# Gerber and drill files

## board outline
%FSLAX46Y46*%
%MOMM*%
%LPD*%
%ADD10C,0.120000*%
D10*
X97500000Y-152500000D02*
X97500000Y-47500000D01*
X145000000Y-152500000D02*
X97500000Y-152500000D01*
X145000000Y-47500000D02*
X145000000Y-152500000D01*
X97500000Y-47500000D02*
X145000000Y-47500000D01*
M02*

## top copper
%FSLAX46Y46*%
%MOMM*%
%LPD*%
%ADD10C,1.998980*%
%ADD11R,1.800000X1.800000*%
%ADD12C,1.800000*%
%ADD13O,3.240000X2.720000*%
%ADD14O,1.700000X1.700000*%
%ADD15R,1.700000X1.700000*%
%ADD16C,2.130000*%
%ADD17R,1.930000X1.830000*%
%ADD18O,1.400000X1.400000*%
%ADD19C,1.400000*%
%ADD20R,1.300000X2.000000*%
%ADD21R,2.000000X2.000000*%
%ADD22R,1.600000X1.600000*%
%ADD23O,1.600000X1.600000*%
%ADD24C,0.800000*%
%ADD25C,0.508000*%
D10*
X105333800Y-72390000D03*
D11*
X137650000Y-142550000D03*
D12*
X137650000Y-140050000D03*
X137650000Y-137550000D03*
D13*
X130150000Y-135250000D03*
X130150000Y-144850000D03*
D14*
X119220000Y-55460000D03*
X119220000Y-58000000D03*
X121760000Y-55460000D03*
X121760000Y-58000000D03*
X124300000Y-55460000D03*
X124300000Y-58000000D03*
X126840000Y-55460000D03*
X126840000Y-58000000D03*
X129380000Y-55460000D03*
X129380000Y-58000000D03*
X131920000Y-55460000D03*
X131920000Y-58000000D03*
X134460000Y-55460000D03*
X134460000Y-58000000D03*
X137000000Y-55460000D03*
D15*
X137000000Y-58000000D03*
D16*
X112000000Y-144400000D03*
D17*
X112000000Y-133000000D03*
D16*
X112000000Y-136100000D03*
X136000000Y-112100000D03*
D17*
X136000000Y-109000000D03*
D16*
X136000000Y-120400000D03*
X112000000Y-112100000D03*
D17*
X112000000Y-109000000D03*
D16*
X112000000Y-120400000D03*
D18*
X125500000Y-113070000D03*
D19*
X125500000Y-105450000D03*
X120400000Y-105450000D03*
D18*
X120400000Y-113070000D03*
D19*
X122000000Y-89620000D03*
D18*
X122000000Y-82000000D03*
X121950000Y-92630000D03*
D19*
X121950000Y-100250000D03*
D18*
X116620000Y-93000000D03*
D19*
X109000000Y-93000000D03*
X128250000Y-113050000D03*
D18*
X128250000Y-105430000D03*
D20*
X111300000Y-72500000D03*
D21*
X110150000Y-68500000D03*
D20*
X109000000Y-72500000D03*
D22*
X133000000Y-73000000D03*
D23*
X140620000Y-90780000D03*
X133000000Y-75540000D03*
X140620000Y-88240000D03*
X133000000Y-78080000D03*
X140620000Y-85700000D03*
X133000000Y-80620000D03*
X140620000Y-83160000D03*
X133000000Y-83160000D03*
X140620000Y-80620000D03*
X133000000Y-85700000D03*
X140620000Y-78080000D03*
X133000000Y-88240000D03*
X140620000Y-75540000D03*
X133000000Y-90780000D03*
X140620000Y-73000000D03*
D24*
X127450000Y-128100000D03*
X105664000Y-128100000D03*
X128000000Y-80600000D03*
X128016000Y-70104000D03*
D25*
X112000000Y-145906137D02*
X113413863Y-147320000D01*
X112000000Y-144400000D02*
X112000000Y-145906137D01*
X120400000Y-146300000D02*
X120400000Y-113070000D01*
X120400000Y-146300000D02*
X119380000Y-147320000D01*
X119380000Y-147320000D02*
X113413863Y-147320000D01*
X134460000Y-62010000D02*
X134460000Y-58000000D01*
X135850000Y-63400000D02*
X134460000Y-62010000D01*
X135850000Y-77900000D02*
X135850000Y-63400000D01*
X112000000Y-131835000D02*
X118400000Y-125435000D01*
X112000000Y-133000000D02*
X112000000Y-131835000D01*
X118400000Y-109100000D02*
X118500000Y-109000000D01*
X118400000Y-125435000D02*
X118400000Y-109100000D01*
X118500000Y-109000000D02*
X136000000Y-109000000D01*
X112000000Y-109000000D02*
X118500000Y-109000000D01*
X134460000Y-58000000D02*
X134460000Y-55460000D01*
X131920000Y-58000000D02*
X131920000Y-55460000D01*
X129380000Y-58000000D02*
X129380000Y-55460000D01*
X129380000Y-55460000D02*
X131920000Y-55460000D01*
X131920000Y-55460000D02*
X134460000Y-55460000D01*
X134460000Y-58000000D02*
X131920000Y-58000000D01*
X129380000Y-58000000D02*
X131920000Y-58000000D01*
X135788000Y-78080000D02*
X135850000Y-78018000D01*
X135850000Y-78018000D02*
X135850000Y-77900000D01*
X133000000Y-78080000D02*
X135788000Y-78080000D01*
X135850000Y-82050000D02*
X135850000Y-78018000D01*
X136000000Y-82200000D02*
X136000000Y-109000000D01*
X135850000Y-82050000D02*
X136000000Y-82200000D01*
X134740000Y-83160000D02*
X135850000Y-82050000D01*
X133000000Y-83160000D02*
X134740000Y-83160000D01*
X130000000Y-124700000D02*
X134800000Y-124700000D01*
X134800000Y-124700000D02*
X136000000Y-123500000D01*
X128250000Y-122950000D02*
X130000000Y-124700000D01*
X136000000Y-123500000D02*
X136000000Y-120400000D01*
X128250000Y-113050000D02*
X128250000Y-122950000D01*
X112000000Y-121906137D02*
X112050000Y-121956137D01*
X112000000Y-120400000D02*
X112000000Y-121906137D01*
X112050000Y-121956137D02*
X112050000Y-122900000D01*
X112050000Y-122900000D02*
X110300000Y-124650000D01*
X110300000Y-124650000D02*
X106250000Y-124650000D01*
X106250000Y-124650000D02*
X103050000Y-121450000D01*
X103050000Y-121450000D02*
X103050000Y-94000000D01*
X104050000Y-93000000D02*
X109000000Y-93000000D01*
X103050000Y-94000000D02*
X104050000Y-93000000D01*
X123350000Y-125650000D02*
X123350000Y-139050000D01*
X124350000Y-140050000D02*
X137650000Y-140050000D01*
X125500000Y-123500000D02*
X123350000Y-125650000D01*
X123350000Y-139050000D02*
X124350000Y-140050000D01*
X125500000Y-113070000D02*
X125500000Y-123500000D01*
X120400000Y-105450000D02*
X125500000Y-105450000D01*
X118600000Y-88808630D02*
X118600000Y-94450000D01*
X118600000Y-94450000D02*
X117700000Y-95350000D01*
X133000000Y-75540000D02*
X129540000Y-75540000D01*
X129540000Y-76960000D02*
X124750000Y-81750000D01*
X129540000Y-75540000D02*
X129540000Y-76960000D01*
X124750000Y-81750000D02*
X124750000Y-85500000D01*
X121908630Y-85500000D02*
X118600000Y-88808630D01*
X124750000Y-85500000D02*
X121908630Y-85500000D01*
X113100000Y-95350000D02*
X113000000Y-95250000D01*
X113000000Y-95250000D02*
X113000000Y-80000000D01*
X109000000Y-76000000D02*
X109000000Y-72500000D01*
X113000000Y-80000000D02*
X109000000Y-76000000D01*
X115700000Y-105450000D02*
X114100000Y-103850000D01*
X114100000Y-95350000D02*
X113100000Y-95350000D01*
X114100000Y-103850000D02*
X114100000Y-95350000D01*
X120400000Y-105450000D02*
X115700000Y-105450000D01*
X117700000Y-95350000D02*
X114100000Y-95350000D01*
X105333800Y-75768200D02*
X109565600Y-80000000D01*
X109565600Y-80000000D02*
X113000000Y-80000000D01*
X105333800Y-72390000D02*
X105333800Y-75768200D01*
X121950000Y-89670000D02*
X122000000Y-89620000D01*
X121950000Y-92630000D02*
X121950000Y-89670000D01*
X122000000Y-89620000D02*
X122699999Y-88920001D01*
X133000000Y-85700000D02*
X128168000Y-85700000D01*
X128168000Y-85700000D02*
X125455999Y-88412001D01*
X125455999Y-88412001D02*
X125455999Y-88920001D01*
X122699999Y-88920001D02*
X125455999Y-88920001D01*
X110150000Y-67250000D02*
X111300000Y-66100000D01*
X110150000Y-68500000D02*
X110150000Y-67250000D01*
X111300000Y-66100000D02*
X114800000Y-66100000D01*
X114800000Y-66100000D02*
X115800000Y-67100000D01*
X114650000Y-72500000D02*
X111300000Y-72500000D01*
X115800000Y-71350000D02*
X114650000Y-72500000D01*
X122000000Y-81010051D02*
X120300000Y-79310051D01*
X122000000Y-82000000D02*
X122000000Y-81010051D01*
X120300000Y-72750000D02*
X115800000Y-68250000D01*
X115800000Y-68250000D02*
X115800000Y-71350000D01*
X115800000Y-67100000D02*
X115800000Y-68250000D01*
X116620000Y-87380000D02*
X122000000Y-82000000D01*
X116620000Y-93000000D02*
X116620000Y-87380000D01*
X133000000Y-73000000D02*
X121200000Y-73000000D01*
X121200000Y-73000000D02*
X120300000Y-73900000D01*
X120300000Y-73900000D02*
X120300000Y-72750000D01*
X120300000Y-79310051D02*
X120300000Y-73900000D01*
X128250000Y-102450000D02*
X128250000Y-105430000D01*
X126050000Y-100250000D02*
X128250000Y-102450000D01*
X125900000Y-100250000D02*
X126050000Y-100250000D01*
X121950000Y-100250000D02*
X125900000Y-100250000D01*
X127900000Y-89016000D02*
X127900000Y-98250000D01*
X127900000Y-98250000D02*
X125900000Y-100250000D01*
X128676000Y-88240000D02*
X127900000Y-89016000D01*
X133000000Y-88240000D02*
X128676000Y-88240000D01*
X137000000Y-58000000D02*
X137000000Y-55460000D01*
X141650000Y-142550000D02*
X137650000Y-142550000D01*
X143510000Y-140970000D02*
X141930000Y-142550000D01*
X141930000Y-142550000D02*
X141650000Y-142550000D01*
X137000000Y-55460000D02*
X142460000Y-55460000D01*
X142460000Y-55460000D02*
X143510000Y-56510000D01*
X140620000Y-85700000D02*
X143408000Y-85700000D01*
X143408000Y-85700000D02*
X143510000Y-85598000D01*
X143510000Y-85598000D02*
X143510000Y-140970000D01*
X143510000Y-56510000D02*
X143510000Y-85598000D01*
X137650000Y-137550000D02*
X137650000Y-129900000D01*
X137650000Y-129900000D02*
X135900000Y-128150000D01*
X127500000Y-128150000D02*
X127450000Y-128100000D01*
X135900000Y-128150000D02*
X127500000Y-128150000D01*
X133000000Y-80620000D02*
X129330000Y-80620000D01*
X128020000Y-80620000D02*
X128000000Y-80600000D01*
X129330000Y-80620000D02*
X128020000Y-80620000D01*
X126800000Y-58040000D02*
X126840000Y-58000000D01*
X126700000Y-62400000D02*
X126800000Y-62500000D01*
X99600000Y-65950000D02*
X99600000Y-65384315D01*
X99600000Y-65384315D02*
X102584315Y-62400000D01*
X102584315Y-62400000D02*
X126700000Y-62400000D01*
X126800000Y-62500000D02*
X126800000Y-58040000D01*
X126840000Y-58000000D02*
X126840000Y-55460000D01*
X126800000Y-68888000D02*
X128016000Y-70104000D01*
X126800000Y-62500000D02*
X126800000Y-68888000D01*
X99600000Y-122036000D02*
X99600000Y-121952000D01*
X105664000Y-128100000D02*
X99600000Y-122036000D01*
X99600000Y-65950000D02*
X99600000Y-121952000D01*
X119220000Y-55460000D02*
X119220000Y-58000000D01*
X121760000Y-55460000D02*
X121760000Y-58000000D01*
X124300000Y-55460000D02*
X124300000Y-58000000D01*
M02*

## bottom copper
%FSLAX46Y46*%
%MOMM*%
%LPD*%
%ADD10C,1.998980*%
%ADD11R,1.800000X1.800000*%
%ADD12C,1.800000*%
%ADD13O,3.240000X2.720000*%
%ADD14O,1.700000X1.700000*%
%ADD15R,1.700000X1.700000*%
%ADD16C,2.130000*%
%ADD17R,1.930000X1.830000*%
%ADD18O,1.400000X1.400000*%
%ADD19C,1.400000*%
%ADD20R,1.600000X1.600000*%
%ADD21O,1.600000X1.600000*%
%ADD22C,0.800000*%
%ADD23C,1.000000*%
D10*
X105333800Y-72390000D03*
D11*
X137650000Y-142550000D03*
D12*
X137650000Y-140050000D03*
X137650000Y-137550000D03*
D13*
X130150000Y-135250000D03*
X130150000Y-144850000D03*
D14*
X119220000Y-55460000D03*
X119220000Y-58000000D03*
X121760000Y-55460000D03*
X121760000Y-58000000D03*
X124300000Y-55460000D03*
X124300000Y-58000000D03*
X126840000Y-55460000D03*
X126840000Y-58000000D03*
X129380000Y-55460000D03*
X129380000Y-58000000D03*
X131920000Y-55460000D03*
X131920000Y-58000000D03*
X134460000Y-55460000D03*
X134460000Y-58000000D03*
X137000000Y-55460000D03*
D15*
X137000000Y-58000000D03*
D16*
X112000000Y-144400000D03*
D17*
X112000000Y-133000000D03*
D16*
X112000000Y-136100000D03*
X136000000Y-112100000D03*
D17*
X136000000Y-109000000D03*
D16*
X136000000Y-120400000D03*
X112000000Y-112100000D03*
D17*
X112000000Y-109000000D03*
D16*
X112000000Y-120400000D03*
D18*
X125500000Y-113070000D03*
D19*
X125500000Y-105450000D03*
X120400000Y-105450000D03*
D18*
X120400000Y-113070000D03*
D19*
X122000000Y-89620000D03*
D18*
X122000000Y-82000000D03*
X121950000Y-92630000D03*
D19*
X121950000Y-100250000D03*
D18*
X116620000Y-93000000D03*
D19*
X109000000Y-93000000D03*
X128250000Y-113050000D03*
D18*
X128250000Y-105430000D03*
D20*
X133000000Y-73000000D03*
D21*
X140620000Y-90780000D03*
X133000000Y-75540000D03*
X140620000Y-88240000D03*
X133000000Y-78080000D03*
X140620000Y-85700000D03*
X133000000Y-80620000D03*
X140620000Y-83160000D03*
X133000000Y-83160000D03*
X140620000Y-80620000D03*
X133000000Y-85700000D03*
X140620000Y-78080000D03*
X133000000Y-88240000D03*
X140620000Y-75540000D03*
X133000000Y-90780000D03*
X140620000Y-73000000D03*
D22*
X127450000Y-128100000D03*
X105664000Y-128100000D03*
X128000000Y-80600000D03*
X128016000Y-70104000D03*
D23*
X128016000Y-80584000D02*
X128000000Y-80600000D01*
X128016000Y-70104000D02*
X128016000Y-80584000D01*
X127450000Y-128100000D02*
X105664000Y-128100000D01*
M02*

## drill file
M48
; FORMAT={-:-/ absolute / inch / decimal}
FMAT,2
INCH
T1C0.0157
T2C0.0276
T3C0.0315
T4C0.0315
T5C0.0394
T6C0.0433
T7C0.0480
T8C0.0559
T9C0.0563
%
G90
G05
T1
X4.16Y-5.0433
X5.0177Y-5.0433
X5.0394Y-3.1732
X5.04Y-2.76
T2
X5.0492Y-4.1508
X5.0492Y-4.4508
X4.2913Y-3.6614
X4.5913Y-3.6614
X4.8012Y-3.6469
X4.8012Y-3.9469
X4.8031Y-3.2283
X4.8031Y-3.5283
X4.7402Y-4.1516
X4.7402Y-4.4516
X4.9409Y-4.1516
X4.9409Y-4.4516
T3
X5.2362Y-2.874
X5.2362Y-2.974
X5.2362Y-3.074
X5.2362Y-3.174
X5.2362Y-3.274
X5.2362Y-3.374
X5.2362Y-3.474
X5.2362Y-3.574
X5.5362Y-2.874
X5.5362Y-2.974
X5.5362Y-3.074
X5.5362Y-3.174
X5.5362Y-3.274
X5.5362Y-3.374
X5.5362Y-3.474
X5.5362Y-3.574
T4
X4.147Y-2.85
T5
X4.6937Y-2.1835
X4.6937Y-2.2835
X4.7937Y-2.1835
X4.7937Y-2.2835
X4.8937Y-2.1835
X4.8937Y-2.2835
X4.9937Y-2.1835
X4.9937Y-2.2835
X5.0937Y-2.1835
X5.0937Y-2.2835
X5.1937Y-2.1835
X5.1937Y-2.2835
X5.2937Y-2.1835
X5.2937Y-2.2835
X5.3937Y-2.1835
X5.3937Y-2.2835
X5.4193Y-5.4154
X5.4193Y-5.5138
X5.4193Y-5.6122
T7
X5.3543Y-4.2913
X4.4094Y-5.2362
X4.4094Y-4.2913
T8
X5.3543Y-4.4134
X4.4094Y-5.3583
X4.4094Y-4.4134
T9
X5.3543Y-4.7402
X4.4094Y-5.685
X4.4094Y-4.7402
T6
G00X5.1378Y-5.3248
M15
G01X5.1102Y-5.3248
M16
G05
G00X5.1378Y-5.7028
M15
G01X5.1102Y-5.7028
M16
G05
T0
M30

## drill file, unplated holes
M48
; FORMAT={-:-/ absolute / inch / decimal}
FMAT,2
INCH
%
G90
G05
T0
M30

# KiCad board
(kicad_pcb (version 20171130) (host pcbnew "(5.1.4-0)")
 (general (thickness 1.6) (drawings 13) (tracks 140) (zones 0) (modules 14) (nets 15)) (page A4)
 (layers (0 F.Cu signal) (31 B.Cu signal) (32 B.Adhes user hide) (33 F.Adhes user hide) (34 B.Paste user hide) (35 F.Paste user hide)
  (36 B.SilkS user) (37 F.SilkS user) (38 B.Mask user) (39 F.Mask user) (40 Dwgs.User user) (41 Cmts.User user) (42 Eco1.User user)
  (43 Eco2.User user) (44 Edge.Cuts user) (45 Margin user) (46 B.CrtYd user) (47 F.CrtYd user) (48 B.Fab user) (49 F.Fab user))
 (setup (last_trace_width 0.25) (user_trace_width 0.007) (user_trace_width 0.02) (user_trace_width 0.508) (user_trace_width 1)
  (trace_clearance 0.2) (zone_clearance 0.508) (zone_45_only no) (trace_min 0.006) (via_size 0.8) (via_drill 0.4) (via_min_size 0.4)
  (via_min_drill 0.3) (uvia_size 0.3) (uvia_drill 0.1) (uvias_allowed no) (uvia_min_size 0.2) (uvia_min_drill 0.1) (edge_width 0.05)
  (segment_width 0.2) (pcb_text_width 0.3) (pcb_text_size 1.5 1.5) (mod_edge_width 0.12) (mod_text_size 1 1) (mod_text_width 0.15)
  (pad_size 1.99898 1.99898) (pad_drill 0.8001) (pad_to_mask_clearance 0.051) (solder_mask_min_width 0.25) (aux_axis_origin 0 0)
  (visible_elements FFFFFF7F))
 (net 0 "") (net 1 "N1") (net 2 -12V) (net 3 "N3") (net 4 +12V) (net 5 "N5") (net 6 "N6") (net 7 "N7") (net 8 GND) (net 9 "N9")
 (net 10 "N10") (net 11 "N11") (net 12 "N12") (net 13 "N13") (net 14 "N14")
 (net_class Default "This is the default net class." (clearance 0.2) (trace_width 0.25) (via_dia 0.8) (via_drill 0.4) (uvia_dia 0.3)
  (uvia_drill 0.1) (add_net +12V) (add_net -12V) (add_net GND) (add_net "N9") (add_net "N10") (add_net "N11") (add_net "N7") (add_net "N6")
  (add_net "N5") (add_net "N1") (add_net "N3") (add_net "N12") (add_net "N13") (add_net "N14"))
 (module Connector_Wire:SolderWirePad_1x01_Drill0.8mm (layer F.Cu) (at 105.3338 72.39)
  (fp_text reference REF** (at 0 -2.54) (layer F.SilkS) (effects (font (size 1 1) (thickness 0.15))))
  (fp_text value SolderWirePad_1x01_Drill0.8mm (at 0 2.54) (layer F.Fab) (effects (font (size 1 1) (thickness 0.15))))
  (pad 1 thru_hole circle (at 0 0) (size 1.99898 1.99898) (drill 0.8001) (layers *.Cu *.Mask) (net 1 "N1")))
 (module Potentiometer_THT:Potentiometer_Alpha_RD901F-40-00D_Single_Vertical (layer F.Cu) (at 137.65 142.55 180)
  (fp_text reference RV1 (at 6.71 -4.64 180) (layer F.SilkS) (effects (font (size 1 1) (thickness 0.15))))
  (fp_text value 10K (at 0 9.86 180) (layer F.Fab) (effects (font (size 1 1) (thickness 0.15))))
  (pad 1 thru_hole rect (at 0 0 270) (size 1.8 1.8) (drill 1) (layers *.Cu *.Mask) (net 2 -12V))
  (pad 2 thru_hole circle (at 0 2.5 270) (size 1.8 1.8) (drill 1) (layers *.Cu *.Mask) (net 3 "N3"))
  (pad 3 thru_hole circle (at 0 5 270) (size 1.8 1.8) (drill 1) (layers *.Cu *.Mask) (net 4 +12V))
  (pad "" thru_hole oval (at 7.5 7.3 270) (size 2.72 3.24) (drill oval 1.1 1.8) (layers *.Cu *.Mask))
  (pad "" thru_hole oval (at 7.5 -2.3 270) (size 2.72 3.24) (drill oval 1.1 1.8) (layers *.Cu *.Mask)))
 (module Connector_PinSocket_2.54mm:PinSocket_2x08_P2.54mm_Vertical (layer F.Cu) (at 137 58 270)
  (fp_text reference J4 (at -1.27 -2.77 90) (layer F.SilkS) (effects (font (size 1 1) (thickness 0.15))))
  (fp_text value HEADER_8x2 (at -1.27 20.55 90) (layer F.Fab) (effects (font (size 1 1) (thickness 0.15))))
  (pad 16 thru_hole oval (at -2.54 17.78 270) (size 1.7 1.7) (drill 1) (layers *.Cu *.Mask) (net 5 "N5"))
  (pad 15 thru_hole oval (at 0 17.78 270) (size 1.7 1.7) (drill 1) (layers *.Cu *.Mask) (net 5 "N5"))
  (pad 14 thru_hole oval (at -2.54 15.24 270) (size 1.7 1.7) (drill 1) (layers *.Cu *.Mask) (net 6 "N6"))
  (pad 13 thru_hole oval (at 0 15.24 270) (size 1.7 1.7) (drill 1) (layers *.Cu *.Mask) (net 6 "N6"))
  (pad 12 thru_hole oval (at -2.54 12.7 270) (size 1.7 1.7) (drill 1) (layers *.Cu *.Mask) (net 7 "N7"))
  (pad 11 thru_hole oval (at 0 12.7 270) (size 1.7 1.7) (drill 1) (layers *.Cu *.Mask) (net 7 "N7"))
  (pad 10 thru_hole oval (at -2.54 10.16 270) (size 1.7 1.7) (drill 1) (layers *.Cu *.Mask) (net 4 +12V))
  (pad 9 thru_hole oval (at 0 10.16 270) (size 1.7 1.7) (drill 1) (layers *.Cu *.Mask) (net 4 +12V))
  (pad 8 thru_hole oval (at -2.54 7.62 270) (size 1.7 1.7) (drill 1) (layers *.Cu *.Mask) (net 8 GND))
  (pad 7 thru_hole oval (at 0 7.62 270) (size 1.7 1.7) (drill 1) (layers *.Cu *.Mask) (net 8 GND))
  (pad 6 thru_hole oval (at -2.54 5.08 270) (size 1.7 1.7) (drill 1) (layers *.Cu *.Mask) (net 8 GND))
  (pad 5 thru_hole oval (at 0 5.08 270) (size 1.7 1.7) (drill 1) (layers *.Cu *.Mask) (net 8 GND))
  (pad 4 thru_hole oval (at -2.54 2.54 270) (size 1.7 1.7) (drill 1) (layers *.Cu *.Mask) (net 8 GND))
  (pad 3 thru_hole oval (at 0 2.54 270) (size 1.7 1.7) (drill 1) (layers *.Cu *.Mask) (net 8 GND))
  (pad 2 thru_hole oval (at -2.54 0 270) (size 1.7 1.7) (drill 1) (layers *.Cu *.Mask) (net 2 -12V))
  (pad 1 thru_hole rect (at 0 0 270) (size 1.7 1.7) (drill 1) (layers *.Cu *.Mask) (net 2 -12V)))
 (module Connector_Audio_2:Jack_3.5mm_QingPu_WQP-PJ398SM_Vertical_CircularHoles (layer F.Cu) (at 112 133)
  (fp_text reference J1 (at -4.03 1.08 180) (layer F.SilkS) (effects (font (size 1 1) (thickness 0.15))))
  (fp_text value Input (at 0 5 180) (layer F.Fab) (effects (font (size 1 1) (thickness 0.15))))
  (pad T thru_hole circle (at 0 11.4 180) (size 2.13 2.13) (drill 1.43) (layers *.Cu *.Mask) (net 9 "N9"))
  (pad S thru_hole rect (at 0 0 180) (size 1.93 1.83) (drill 1.22) (layers *.Cu *.Mask) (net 8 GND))
  (pad TN thru_hole circle (at 0 3.1 180) (size 2.13 2.13) (drill 1.42) (layers *.Cu *.Mask)))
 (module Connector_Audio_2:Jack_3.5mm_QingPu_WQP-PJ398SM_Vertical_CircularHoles (layer F.Cu) (at 136 109)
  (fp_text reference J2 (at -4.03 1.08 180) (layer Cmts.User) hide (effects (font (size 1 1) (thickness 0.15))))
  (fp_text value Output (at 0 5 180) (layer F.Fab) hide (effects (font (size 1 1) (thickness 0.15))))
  (pad TN thru_hole circle (at 0 3.1 180) (size 2.13 2.13) (drill 1.42) (layers *.Cu *.Mask))
  (pad S thru_hole rect (at 0 0 180) (size 1.93 1.83) (drill 1.22) (layers *.Cu *.Mask) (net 8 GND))
  (pad T thru_hole circle (at 0 11.4 180) (size 2.13 2.13) (drill 1.43) (layers *.Cu *.Mask) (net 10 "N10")))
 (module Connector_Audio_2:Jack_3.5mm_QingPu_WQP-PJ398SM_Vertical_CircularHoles (layer F.Cu) (at 112 109)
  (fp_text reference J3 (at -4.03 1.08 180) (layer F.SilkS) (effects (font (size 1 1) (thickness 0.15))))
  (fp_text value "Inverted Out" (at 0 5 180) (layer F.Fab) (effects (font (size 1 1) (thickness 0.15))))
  (pad TN thru_hole circle (at 0 3.1 180) (size 2.13 2.13) (drill 1.42) (layers *.Cu *.Mask))
  (pad S thru_hole rect (at 0 0 180) (size 1.93 1.83) (drill 1.22) (layers *.Cu *.Mask) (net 8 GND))
  (pad T thru_hole circle (at 0 11.4 180) (size 2.13 2.13) (drill 1.43) (layers *.Cu *.Mask) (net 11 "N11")))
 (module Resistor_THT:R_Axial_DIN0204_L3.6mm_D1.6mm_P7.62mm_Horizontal (layer F.Cu) (at 125.5 105.45 270)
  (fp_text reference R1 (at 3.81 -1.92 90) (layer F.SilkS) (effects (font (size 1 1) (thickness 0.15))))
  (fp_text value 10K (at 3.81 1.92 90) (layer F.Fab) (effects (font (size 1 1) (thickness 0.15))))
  (pad 2 thru_hole oval (at 7.62 0 270) (size 1.4 1.4) (drill 0.7) (layers *.Cu *.Mask) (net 3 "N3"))
  (pad 1 thru_hole circle (at 0 0 270) (size 1.4 1.4) (drill 0.7) (layers *.Cu *.Mask) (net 1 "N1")))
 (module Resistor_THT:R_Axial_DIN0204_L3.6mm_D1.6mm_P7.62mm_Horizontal (layer F.Cu) (at 120.4 105.45 270)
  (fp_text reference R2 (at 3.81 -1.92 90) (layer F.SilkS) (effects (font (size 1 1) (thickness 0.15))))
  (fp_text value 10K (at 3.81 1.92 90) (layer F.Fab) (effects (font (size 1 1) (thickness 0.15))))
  (pad 1 thru_hole circle (at 0 0 270) (size 1.4 1.4) (drill 0.7) (layers *.Cu *.Mask) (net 1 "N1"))
  (pad 2 thru_hole oval (at 7.62 0 270) (size 1.4 1.4) (drill 0.7) (layers *.Cu *.Mask) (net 9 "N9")))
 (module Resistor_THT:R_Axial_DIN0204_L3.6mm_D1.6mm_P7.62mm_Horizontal (layer F.Cu) (at 122 89.62 90)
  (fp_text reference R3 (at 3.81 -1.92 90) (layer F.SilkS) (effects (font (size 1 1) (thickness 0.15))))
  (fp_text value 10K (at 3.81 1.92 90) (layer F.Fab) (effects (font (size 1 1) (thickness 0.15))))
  (pad 1 thru_hole circle (at 0 0 90) (size 1.4 1.4) (drill 0.7) (layers *.Cu *.Mask) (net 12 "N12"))
  (pad 2 thru_hole oval (at 7.62 0 90) (size 1.4 1.4) (drill 0.7) (layers *.Cu *.Mask) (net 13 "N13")))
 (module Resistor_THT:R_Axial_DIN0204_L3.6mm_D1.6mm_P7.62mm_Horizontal (layer F.Cu) (at 121.95 100.25 90)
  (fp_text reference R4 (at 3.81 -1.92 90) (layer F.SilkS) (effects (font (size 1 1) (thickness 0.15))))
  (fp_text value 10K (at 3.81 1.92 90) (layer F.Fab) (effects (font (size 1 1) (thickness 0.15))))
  (pad 2 thru_hole oval (at 7.62 0 90) (size 1.4 1.4) (drill 0.7) (layers *.Cu *.Mask) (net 12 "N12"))
  (pad 1 thru_hole circle (at 0 0 90) (size 1.4 1.4) (drill 0.7) (layers *.Cu *.Mask) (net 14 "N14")))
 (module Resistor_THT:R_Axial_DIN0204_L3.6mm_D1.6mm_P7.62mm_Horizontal (layer F.Cu) (at 109 93)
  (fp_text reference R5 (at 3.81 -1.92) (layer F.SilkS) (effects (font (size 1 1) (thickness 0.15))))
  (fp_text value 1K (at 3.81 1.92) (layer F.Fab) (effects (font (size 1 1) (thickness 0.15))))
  (pad 2 thru_hole oval (at 7.62 0) (size 1.4 1.4) (drill 0.7) (layers *.Cu *.Mask) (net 13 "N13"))
  (pad 1 thru_hole circle (at 0 0) (size 1.4 1.4) (drill 0.7) (layers *.Cu *.Mask) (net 11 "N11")))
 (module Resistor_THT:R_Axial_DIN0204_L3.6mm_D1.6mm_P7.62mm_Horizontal (layer F.Cu) (at 128.25 113.05 90)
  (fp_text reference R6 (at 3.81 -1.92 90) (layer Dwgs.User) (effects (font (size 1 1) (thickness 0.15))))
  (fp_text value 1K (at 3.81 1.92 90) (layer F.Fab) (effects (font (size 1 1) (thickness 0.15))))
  (pad 1 thru_hole circle (at 0 0 90) (size 1.4 1.4) (drill 0.7) (layers *.Cu *.Mask) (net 10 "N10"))
  (pad 2 thru_hole oval (at 7.62 0 90) (size 1.4 1.4) (drill 0.7) (layers *.Cu *.Mask) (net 14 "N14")))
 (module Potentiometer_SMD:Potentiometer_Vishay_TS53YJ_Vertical (layer F.Cu) (at 110.15 70.5 270)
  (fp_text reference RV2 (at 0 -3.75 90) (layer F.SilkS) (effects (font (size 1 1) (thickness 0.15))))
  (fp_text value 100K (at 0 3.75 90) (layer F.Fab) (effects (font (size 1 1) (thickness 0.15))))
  (pad 1 smd rect (at 2 -1.15 270) (size 2 1.3) (layers F.Cu F.Paste F.Mask) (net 13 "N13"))
  (pad 2 smd rect (at -2 0 270) (size 2 2) (layers F.Cu F.Paste F.Mask) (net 13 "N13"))
  (pad 3 smd rect (at 2 1.15 270) (size 2 1.3) (layers F.Cu F.Paste F.Mask) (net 1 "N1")))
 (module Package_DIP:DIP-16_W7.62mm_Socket (layer F.Cu) (at 133 73)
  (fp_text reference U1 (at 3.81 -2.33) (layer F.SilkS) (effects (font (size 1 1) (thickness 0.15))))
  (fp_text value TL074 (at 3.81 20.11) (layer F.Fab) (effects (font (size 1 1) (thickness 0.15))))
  (pad 1 thru_hole rect (at 0 0) (size 1.6 1.6) (drill 0.8) (layers *.Cu *.Mask) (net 13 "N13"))
  (pad 9 thru_hole oval (at 7.62 17.78) (size 1.6 1.6) (drill 0.8) (layers *.Cu *.Mask))
  (pad 2 thru_hole oval (at 0 2.54) (size 1.6 1.6) (drill 0.8) (layers *.Cu *.Mask) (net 1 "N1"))
  (pad 10 thru_hole oval (at 7.62 15.24) (size 1.6 1.6) (drill 0.8) (layers *.Cu *.Mask))
  (pad 3 thru_hole oval (at 0 5.08) (size 1.6 1.6) (drill 0.8) (layers *.Cu *.Mask) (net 8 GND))
  (pad 11 thru_hole oval (at 7.62 12.7) (size 1.6 1.6) (drill 0.8) (layers *.Cu *.Mask) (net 2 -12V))
  (pad 4 thru_hole oval (at 0 7.62) (size 1.6 1.6) (drill 0.8) (layers *.Cu *.Mask) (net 4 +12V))
  (pad 12 thru_hole oval (at 7.62 10.16) (size 1.6 1.6) (drill 0.8) (layers *.Cu *.Mask))
  (pad 5 thru_hole oval (at 0 10.16) (size 1.6 1.6) (drill 0.8) (layers *.Cu *.Mask) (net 8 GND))
  (pad 13 thru_hole oval (at 7.62 7.62) (size 1.6 1.6) (drill 0.8) (layers *.Cu *.Mask))
  (pad 6 thru_hole oval (at 0 12.7) (size 1.6 1.6) (drill 0.8) (layers *.Cu *.Mask) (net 12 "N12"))
  (pad 14 thru_hole oval (at 7.62 5.08) (size 1.6 1.6) (drill 0.8) (layers *.Cu *.Mask))
  (pad 7 thru_hole oval (at 0 15.24) (size 1.6 1.6) (drill 0.8) (layers *.Cu *.Mask) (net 14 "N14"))
  (pad 15 thru_hole oval (at 7.62 2.54) (size 1.6 1.6) (drill 0.8) (layers *.Cu *.Mask))
  (pad 8 thru_hole oval (at 0 17.78) (size 1.6 1.6) (drill 0.8) (layers *.Cu *.Mask))
  (pad 16 thru_hole oval (at 7.62 0) (size 1.6 1.6) (drill 0.8) (layers *.Cu *.Mask)))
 (gr_line (start 97.5 152.5) (end 97.5 47.5) (layer Edge.Cuts) (width 0.12))
 (gr_line (start 145 152.5) (end 97.5 152.5) (layer Edge.Cuts) (width 0.12))
 (gr_line (start 145 47.5) (end 145 152.5) (layer Edge.Cuts) (width 0.12))
 (gr_line (start 97.5 47.5) (end 145 47.5) (layer Edge.Cuts) (width 0.12))
 (segment (start 112 145.906137) (end 113.413863 147.32) (width 0.508) (layer F.Cu) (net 9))
 (segment (start 112 144.4) (end 112 145.906137) (width 0.508) (layer F.Cu) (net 9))
 (segment (start 120.4 146.3) (end 120.4 113.07) (width 0.508) (layer F.Cu) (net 9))
 (segment (start 120.4 146.3) (end 119.38 147.32) (width 0.508) (layer F.Cu) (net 9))
 (segment (start 119.38 147.32) (end 113.413863 147.32) (width 0.508) (layer F.Cu) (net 9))
 (segment (start 134.46 62.01) (end 134.46 58) (width 0.508) (layer F.Cu) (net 8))
 (segment (start 135.85 63.4) (end 134.46 62.01) (width 0.508) (layer F.Cu) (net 8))
 (segment (start 135.85 77.9) (end 135.85 63.4) (width 0.508) (layer F.Cu) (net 8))
 (segment (start 112 131.835) (end 118.4 125.435) (width 0.508) (layer F.Cu) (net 8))
 (segment (start 112 133) (end 112 131.835) (width 0.508) (layer F.Cu) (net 8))
 (segment (start 118.4 109.1) (end 118.5 109) (width 0.508) (layer F.Cu) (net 8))
 (segment (start 118.4 125.435) (end 118.4 109.1) (width 0.508) (layer F.Cu) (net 8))
 (segment (start 118.5 109) (end 136 109) (width 0.508) (layer F.Cu) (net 8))
 (segment (start 112 109) (end 118.5 109) (width 0.508) (layer F.Cu) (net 8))
 (segment (start 134.46 58) (end 134.46 55.46) (width 0.508) (layer F.Cu) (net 8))
 (segment (start 131.92 58) (end 131.92 55.46) (width 0.508) (layer F.Cu) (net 8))
 (segment (start 129.38 58) (end 129.38 55.46) (width 0.508) (layer F.Cu) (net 8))
 (segment (start 129.38 55.46) (end 131.92 55.46) (width 0.508) (layer F.Cu) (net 8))
 (segment (start 131.92 55.46) (end 134.46 55.46) (width 0.508) (layer F.Cu) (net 8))
 (segment (start 134.46 58) (end 131.92 58) (width 0.508) (layer F.Cu) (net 8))
 (segment (start 129.38 58) (end 131.92 58) (width 0.508) (layer F.Cu) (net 8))
 (segment (start 135.788 78.08) (end 135.85 78.018) (width 0.508) (layer F.Cu) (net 8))
 (segment (start 135.85 78.018) (end 135.85 77.9) (width 0.508) (layer F.Cu) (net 8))
 (segment (start 133 78.08) (end 135.788 78.08) (width 0.508) (layer F.Cu) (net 8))
 (segment (start 135.85 82.05) (end 135.85 78.018) (width 0.508) (layer F.Cu) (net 8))
 (segment (start 136 82.2) (end 136 109) (width 0.508) (layer F.Cu) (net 8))
 (segment (start 135.85 82.05) (end 136 82.2) (width 0.508) (layer F.Cu) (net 8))
 (segment (start 134.74 83.16) (end 135.85 82.05) (width 0.508) (layer F.Cu) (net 8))
 (segment (start 133 83.16) (end 134.74 83.16) (width 0.508) (layer F.Cu) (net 8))
 (segment (start 130 124.7) (end 134.8 124.7) (width 0.508) (layer F.Cu) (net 10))
 (segment (start 134.8 124.7) (end 136 123.5) (width 0.508) (layer F.Cu) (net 10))
 (segment (start 128.25 122.95) (end 130 124.7) (width 0.508) (layer F.Cu) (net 10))
 (segment (start 136 123.5) (end 136 120.4) (width 0.508) (layer F.Cu) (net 10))
 (segment (start 128.25 113.05) (end 128.25 122.95) (width 0.508) (layer F.Cu) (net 10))
 (segment (start 112 121.906137) (end 112.05 121.956137) (width 0.508) (layer F.Cu) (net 11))
 (segment (start 112 120.4) (end 112 121.906137) (width 0.508) (layer F.Cu) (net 11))
 (segment (start 112.05 121.956137) (end 112.05 122.9) (width 0.508) (layer F.Cu) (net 11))
 (segment (start 112.05 122.9) (end 110.3 124.65) (width 0.508) (layer F.Cu) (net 11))
 (segment (start 110.3 124.65) (end 106.25 124.65) (width 0.508) (layer F.Cu) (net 11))
 (segment (start 106.25 124.65) (end 103.05 121.45) (width 0.508) (layer F.Cu) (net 11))
 (segment (start 103.05 121.45) (end 103.05 94) (width 0.508) (layer F.Cu) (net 11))
 (segment (start 104.05 93) (end 109 93) (width 0.508) (layer F.Cu) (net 11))
 (segment (start 103.05 94) (end 104.05 93) (width 0.508) (layer F.Cu) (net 11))
 (segment (start 123.35 125.65) (end 123.35 139.05) (width 0.508) (layer F.Cu) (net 3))
 (segment (start 124.35 140.05) (end 137.65 140.05) (width 0.508) (layer F.Cu) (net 3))
 (segment (start 125.5 123.5) (end 123.35 125.65) (width 0.508) (layer F.Cu) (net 3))
 (segment (start 123.35 139.05) (end 124.35 140.05) (width 0.508) (layer F.Cu) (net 3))
 (segment (start 125.5 113.07) (end 125.5 123.5) (width 0.508) (layer F.Cu) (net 3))
 (segment (start 120.4 105.45) (end 125.5 105.45) (width 0.508) (layer F.Cu) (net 1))
 (segment (start 118.6 88.80863) (end 118.6 94.45) (width 0.508) (layer F.Cu) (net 1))
 (segment (start 118.6 94.45) (end 117.7 95.35) (width 0.508) (layer F.Cu) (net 1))
 (segment (start 133 75.54) (end 129.54 75.54) (width 0.508) (layer F.Cu) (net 1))
 (segment (start 129.54 76.96) (end 124.75 81.75) (width 0.508) (layer F.Cu) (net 1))
 (segment (start 129.54 75.54) (end 129.54 76.96) (width 0.508) (layer F.Cu) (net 1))
 (segment (start 124.75 81.75) (end 124.75 85.5) (width 0.508) (layer F.Cu) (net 1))
 (segment (start 121.90863 85.5) (end 118.6 88.80863) (width 0.508) (layer F.Cu) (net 1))
 (segment (start 124.75 85.5) (end 121.90863 85.5) (width 0.508) (layer F.Cu) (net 1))
 (segment (start 113.1 95.35) (end 113 95.25) (width 0.508) (layer F.Cu) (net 1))
 (segment (start 113 95.25) (end 113 80) (width 0.508) (layer F.Cu) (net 1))
 (segment (start 109 76) (end 109 72.5) (width 0.508) (layer F.Cu) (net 1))
 (segment (start 113 80) (end 109 76) (width 0.508) (layer F.Cu) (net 1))
 (segment (start 115.7 105.45) (end 114.1 103.85) (width 0.508) (layer F.Cu) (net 1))
 (segment (start 114.1 95.35) (end 113.1 95.35) (width 0.508) (layer F.Cu) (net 1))
 (segment (start 114.1 103.85) (end 114.1 95.35) (width 0.508) (layer F.Cu) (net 1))
 (segment (start 120.4 105.45) (end 115.7 105.45) (width 0.508) (layer F.Cu) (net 1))
 (segment (start 117.7 95.35) (end 114.1 95.35) (width 0.508) (layer F.Cu) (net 1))
 (segment (start 105.3338 75.7682) (end 109.5656 80) (width 0.508) (layer F.Cu) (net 1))
 (segment (start 109.5656 80) (end 113 80) (width 0.508) (layer F.Cu) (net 1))
 (segment (start 105.3338 72.39) (end 105.3338 75.7682) (width 0.508) (layer F.Cu) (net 1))
 (segment (start 121.95 89.67) (end 122 89.62) (width 0.508) (layer F.Cu) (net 12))
 (segment (start 121.95 92.63) (end 121.95 89.67) (width 0.508) (layer F.Cu) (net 12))
 (segment (start 122 89.62) (end 122.699999 88.920001) (width 0.508) (layer F.Cu) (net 12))
 (segment (start 133 85.7) (end 128.168 85.7) (width 0.508) (layer F.Cu) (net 12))
 (segment (start 128.168 85.7) (end 125.455999 88.412001) (width 0.508) (layer F.Cu) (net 12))
 (segment (start 125.455999 88.412001) (end 125.455999 88.920001) (width 0.508) (layer F.Cu) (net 12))
 (segment (start 122.699999 88.920001) (end 125.455999 88.920001) (width 0.508) (layer F.Cu) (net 12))
 (segment (start 110.15 67.25) (end 111.3 66.1) (width 0.508) (layer F.Cu) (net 13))
 (segment (start 110.15 68.5) (end 110.15 67.25) (width 0.508) (layer F.Cu) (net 13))
 (segment (start 111.3 66.1) (end 114.8 66.1) (width 0.508) (layer F.Cu) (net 13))
 (segment (start 114.8 66.1) (end 115.8 67.1) (width 0.508) (layer F.Cu) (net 13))
 (segment (start 114.65 72.5) (end 111.3 72.5) (width 0.508) (layer F.Cu) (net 13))
 (segment (start 115.8 71.35) (end 114.65 72.5) (width 0.508) (layer F.Cu) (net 13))
 (segment (start 122 81.010051) (end 120.3 79.310051) (width 0.508) (layer F.Cu) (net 13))
 (segment (start 122 82) (end 122 81.010051) (width 0.508) (layer F.Cu) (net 13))
 (segment (start 120.3 72.75) (end 115.8 68.25) (width 0.508) (layer F.Cu) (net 13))
 (segment (start 115.8 68.25) (end 115.8 71.35) (width 0.508) (layer F.Cu) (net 13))
 (segment (start 115.8 67.1) (end 115.8 68.25) (width 0.508) (layer F.Cu) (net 13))
 (segment (start 116.62 87.38) (end 122 82) (width 0.508) (layer F.Cu) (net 13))
 (segment (start 116.62 93) (end 116.62 87.38) (width 0.508) (layer F.Cu) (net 13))
 (segment (start 133 73) (end 121.2 73) (width 0.508) (layer F.Cu) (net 13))
 (segment (start 121.2 73) (end 120.3 73.9) (width 0.508) (layer F.Cu) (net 13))
 (segment (start 120.3 73.9) (end 120.3 72.75) (width 0.508) (layer F.Cu) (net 13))
 (segment (start 120.3 79.310051) (end 120.3 73.9) (width 0.508) (layer F.Cu) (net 13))
 (segment (start 128.25 102.45) (end 128.25 105.43) (width 0.508) (layer F.Cu) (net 14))
 (segment (start 126.05 100.25) (end 128.25 102.45) (width 0.508) (layer F.Cu) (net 14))
 (segment (start 125.9 100.25) (end 126.05 100.25) (width 0.508) (layer F.Cu) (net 14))
 (segment (start 121.95 100.25) (end 125.9 100.25) (width 0.508) (layer F.Cu) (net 14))
 (segment (start 127.9 89.016) (end 127.9 98.25) (width 0.508) (layer F.Cu) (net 14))
 (segment (start 127.9 98.25) (end 125.9 100.25) (width 0.508) (layer F.Cu) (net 14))
 (segment (start 128.676 88.24) (end 127.9 89.016) (width 0.508) (layer F.Cu) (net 14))
 (segment (start 133 88.24) (end 128.676 88.24) (width 0.508) (layer F.Cu) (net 14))
 (segment (start 137 58) (end 137 55.46) (width 0.508) (layer F.Cu) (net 2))
 (segment (start 141.65 142.55) (end 137.65 142.55) (width 0.508) (layer F.Cu) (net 2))
 (segment (start 143.51 140.97) (end 141.93 142.55) (width 0.508) (layer F.Cu) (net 2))
 (segment (start 141.93 142.55) (end 141.65 142.55) (width 0.508) (layer F.Cu) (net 2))
 (segment (start 137 55.46) (end 142.46 55.46) (width 0.508) (layer F.Cu) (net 2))
 (segment (start 142.46 55.46) (end 143.51 56.51) (width 0.508) (layer F.Cu) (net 2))
 (segment (start 140.62 85.7) (end 143.408 85.7) (width 0.508) (layer F.Cu) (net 2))
 (segment (start 143.408 85.7) (end 143.51 85.598) (width 0.508) (layer F.Cu) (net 2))
 (segment (start 143.51 85.598) (end 143.51 140.97) (width 0.508) (layer F.Cu) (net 2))
 (segment (start 143.51 56.51) (end 143.51 85.598) (width 0.508) (layer F.Cu) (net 2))
 (segment (start 137.65 137.55) (end 137.65 129.9) (width 0.508) (layer F.Cu) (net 4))
 (segment (start 137.65 129.9) (end 135.9 128.15) (width 0.508) (layer F.Cu) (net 4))
 (via (at 127.45 128.1) (size 0.8) (drill 0.4) (layers F.Cu B.Cu) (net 4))
 (segment (start 127.5 128.15) (end 127.45 128.1) (width 0.508) (layer F.Cu) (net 4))
 (segment (start 135.9 128.15) (end 127.5 128.15) (width 0.508) (layer F.Cu) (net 4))
 (via (at 105.664 128.1) (size 0.8) (drill 0.4) (layers F.Cu B.Cu) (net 4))
 (segment (start 133 80.62) (end 129.33 80.62) (width 0.508) (layer F.Cu) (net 4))
 (segment (start 128.02 80.62) (end 128 80.6) (width 0.508) (layer F.Cu) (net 4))
 (via (at 128 80.6) (size 0.8) (drill 0.4) (layers F.Cu B.Cu) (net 4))
 (segment (start 129.33 80.62) (end 128.02 80.62) (width 0.508) (layer F.Cu) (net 4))
 (via (at 128.016 70.104) (size 0.8) (drill 0.4) (layers F.Cu B.Cu) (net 4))
 (segment (start 126.8 58.04) (end 126.84 58) (width 0.508) (layer F.Cu) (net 4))
 (segment (start 126.7 62.4) (end 126.8 62.5) (width 0.508) (layer F.Cu) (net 4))
 (segment (start 99.6 65.95) (end 99.6 65.384315) (width 0.508) (layer F.Cu) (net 4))
 (segment (start 99.6 65.384315) (end 102.584315 62.4) (width 0.508) (layer F.Cu) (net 4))
 (segment (start 102.584315 62.4) (end 126.7 62.4) (width 0.508) (layer F.Cu) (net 4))
 (segment (start 126.8 62.5) (end 126.8 58.04) (width 0.508) (layer F.Cu) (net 4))
 (segment (start 126.84 58) (end 126.84 55.46) (width 0.508) (layer F.Cu) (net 4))
 (segment (start 126.8 68.888) (end 128.016 70.104) (width 0.508) (layer F.Cu) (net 4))
 (segment (start 126.8 62.5) (end 126.8 68.888) (width 0.508) (layer F.Cu) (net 4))
 (segment (start 128.016 80.584) (end 128 80.6) (width 1) (layer B.Cu) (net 4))
 (segment (start 128.016 70.104) (end 128.016 80.584) (width 1) (layer B.Cu) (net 4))
 (segment (start 127.45 128.1) (end 105.664 128.1) (width 1) (layer B.Cu) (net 4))
 (segment (start 99.6 122.036) (end 99.6 121.952) (width 0.508) (layer F.Cu) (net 4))
 (segment (start 105.664 128.1) (end 99.6 122.036) (width 0.508) (layer F.Cu) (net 4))
 (segment (start 99.6 65.95) (end 99.6 121.952) (width 0.508) (layer F.Cu) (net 4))
 (segment (start 119.22 55.46) (end 119.22 58) (width 0.508) (layer F.Cu) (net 5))
 (segment (start 121.76 55.46) (end 121.76 58) (width 0.508) (layer F.Cu) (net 6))
 (segment (start 124.3 55.46) (end 124.3 58) (width 0.508) (layer F.Cu) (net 7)))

